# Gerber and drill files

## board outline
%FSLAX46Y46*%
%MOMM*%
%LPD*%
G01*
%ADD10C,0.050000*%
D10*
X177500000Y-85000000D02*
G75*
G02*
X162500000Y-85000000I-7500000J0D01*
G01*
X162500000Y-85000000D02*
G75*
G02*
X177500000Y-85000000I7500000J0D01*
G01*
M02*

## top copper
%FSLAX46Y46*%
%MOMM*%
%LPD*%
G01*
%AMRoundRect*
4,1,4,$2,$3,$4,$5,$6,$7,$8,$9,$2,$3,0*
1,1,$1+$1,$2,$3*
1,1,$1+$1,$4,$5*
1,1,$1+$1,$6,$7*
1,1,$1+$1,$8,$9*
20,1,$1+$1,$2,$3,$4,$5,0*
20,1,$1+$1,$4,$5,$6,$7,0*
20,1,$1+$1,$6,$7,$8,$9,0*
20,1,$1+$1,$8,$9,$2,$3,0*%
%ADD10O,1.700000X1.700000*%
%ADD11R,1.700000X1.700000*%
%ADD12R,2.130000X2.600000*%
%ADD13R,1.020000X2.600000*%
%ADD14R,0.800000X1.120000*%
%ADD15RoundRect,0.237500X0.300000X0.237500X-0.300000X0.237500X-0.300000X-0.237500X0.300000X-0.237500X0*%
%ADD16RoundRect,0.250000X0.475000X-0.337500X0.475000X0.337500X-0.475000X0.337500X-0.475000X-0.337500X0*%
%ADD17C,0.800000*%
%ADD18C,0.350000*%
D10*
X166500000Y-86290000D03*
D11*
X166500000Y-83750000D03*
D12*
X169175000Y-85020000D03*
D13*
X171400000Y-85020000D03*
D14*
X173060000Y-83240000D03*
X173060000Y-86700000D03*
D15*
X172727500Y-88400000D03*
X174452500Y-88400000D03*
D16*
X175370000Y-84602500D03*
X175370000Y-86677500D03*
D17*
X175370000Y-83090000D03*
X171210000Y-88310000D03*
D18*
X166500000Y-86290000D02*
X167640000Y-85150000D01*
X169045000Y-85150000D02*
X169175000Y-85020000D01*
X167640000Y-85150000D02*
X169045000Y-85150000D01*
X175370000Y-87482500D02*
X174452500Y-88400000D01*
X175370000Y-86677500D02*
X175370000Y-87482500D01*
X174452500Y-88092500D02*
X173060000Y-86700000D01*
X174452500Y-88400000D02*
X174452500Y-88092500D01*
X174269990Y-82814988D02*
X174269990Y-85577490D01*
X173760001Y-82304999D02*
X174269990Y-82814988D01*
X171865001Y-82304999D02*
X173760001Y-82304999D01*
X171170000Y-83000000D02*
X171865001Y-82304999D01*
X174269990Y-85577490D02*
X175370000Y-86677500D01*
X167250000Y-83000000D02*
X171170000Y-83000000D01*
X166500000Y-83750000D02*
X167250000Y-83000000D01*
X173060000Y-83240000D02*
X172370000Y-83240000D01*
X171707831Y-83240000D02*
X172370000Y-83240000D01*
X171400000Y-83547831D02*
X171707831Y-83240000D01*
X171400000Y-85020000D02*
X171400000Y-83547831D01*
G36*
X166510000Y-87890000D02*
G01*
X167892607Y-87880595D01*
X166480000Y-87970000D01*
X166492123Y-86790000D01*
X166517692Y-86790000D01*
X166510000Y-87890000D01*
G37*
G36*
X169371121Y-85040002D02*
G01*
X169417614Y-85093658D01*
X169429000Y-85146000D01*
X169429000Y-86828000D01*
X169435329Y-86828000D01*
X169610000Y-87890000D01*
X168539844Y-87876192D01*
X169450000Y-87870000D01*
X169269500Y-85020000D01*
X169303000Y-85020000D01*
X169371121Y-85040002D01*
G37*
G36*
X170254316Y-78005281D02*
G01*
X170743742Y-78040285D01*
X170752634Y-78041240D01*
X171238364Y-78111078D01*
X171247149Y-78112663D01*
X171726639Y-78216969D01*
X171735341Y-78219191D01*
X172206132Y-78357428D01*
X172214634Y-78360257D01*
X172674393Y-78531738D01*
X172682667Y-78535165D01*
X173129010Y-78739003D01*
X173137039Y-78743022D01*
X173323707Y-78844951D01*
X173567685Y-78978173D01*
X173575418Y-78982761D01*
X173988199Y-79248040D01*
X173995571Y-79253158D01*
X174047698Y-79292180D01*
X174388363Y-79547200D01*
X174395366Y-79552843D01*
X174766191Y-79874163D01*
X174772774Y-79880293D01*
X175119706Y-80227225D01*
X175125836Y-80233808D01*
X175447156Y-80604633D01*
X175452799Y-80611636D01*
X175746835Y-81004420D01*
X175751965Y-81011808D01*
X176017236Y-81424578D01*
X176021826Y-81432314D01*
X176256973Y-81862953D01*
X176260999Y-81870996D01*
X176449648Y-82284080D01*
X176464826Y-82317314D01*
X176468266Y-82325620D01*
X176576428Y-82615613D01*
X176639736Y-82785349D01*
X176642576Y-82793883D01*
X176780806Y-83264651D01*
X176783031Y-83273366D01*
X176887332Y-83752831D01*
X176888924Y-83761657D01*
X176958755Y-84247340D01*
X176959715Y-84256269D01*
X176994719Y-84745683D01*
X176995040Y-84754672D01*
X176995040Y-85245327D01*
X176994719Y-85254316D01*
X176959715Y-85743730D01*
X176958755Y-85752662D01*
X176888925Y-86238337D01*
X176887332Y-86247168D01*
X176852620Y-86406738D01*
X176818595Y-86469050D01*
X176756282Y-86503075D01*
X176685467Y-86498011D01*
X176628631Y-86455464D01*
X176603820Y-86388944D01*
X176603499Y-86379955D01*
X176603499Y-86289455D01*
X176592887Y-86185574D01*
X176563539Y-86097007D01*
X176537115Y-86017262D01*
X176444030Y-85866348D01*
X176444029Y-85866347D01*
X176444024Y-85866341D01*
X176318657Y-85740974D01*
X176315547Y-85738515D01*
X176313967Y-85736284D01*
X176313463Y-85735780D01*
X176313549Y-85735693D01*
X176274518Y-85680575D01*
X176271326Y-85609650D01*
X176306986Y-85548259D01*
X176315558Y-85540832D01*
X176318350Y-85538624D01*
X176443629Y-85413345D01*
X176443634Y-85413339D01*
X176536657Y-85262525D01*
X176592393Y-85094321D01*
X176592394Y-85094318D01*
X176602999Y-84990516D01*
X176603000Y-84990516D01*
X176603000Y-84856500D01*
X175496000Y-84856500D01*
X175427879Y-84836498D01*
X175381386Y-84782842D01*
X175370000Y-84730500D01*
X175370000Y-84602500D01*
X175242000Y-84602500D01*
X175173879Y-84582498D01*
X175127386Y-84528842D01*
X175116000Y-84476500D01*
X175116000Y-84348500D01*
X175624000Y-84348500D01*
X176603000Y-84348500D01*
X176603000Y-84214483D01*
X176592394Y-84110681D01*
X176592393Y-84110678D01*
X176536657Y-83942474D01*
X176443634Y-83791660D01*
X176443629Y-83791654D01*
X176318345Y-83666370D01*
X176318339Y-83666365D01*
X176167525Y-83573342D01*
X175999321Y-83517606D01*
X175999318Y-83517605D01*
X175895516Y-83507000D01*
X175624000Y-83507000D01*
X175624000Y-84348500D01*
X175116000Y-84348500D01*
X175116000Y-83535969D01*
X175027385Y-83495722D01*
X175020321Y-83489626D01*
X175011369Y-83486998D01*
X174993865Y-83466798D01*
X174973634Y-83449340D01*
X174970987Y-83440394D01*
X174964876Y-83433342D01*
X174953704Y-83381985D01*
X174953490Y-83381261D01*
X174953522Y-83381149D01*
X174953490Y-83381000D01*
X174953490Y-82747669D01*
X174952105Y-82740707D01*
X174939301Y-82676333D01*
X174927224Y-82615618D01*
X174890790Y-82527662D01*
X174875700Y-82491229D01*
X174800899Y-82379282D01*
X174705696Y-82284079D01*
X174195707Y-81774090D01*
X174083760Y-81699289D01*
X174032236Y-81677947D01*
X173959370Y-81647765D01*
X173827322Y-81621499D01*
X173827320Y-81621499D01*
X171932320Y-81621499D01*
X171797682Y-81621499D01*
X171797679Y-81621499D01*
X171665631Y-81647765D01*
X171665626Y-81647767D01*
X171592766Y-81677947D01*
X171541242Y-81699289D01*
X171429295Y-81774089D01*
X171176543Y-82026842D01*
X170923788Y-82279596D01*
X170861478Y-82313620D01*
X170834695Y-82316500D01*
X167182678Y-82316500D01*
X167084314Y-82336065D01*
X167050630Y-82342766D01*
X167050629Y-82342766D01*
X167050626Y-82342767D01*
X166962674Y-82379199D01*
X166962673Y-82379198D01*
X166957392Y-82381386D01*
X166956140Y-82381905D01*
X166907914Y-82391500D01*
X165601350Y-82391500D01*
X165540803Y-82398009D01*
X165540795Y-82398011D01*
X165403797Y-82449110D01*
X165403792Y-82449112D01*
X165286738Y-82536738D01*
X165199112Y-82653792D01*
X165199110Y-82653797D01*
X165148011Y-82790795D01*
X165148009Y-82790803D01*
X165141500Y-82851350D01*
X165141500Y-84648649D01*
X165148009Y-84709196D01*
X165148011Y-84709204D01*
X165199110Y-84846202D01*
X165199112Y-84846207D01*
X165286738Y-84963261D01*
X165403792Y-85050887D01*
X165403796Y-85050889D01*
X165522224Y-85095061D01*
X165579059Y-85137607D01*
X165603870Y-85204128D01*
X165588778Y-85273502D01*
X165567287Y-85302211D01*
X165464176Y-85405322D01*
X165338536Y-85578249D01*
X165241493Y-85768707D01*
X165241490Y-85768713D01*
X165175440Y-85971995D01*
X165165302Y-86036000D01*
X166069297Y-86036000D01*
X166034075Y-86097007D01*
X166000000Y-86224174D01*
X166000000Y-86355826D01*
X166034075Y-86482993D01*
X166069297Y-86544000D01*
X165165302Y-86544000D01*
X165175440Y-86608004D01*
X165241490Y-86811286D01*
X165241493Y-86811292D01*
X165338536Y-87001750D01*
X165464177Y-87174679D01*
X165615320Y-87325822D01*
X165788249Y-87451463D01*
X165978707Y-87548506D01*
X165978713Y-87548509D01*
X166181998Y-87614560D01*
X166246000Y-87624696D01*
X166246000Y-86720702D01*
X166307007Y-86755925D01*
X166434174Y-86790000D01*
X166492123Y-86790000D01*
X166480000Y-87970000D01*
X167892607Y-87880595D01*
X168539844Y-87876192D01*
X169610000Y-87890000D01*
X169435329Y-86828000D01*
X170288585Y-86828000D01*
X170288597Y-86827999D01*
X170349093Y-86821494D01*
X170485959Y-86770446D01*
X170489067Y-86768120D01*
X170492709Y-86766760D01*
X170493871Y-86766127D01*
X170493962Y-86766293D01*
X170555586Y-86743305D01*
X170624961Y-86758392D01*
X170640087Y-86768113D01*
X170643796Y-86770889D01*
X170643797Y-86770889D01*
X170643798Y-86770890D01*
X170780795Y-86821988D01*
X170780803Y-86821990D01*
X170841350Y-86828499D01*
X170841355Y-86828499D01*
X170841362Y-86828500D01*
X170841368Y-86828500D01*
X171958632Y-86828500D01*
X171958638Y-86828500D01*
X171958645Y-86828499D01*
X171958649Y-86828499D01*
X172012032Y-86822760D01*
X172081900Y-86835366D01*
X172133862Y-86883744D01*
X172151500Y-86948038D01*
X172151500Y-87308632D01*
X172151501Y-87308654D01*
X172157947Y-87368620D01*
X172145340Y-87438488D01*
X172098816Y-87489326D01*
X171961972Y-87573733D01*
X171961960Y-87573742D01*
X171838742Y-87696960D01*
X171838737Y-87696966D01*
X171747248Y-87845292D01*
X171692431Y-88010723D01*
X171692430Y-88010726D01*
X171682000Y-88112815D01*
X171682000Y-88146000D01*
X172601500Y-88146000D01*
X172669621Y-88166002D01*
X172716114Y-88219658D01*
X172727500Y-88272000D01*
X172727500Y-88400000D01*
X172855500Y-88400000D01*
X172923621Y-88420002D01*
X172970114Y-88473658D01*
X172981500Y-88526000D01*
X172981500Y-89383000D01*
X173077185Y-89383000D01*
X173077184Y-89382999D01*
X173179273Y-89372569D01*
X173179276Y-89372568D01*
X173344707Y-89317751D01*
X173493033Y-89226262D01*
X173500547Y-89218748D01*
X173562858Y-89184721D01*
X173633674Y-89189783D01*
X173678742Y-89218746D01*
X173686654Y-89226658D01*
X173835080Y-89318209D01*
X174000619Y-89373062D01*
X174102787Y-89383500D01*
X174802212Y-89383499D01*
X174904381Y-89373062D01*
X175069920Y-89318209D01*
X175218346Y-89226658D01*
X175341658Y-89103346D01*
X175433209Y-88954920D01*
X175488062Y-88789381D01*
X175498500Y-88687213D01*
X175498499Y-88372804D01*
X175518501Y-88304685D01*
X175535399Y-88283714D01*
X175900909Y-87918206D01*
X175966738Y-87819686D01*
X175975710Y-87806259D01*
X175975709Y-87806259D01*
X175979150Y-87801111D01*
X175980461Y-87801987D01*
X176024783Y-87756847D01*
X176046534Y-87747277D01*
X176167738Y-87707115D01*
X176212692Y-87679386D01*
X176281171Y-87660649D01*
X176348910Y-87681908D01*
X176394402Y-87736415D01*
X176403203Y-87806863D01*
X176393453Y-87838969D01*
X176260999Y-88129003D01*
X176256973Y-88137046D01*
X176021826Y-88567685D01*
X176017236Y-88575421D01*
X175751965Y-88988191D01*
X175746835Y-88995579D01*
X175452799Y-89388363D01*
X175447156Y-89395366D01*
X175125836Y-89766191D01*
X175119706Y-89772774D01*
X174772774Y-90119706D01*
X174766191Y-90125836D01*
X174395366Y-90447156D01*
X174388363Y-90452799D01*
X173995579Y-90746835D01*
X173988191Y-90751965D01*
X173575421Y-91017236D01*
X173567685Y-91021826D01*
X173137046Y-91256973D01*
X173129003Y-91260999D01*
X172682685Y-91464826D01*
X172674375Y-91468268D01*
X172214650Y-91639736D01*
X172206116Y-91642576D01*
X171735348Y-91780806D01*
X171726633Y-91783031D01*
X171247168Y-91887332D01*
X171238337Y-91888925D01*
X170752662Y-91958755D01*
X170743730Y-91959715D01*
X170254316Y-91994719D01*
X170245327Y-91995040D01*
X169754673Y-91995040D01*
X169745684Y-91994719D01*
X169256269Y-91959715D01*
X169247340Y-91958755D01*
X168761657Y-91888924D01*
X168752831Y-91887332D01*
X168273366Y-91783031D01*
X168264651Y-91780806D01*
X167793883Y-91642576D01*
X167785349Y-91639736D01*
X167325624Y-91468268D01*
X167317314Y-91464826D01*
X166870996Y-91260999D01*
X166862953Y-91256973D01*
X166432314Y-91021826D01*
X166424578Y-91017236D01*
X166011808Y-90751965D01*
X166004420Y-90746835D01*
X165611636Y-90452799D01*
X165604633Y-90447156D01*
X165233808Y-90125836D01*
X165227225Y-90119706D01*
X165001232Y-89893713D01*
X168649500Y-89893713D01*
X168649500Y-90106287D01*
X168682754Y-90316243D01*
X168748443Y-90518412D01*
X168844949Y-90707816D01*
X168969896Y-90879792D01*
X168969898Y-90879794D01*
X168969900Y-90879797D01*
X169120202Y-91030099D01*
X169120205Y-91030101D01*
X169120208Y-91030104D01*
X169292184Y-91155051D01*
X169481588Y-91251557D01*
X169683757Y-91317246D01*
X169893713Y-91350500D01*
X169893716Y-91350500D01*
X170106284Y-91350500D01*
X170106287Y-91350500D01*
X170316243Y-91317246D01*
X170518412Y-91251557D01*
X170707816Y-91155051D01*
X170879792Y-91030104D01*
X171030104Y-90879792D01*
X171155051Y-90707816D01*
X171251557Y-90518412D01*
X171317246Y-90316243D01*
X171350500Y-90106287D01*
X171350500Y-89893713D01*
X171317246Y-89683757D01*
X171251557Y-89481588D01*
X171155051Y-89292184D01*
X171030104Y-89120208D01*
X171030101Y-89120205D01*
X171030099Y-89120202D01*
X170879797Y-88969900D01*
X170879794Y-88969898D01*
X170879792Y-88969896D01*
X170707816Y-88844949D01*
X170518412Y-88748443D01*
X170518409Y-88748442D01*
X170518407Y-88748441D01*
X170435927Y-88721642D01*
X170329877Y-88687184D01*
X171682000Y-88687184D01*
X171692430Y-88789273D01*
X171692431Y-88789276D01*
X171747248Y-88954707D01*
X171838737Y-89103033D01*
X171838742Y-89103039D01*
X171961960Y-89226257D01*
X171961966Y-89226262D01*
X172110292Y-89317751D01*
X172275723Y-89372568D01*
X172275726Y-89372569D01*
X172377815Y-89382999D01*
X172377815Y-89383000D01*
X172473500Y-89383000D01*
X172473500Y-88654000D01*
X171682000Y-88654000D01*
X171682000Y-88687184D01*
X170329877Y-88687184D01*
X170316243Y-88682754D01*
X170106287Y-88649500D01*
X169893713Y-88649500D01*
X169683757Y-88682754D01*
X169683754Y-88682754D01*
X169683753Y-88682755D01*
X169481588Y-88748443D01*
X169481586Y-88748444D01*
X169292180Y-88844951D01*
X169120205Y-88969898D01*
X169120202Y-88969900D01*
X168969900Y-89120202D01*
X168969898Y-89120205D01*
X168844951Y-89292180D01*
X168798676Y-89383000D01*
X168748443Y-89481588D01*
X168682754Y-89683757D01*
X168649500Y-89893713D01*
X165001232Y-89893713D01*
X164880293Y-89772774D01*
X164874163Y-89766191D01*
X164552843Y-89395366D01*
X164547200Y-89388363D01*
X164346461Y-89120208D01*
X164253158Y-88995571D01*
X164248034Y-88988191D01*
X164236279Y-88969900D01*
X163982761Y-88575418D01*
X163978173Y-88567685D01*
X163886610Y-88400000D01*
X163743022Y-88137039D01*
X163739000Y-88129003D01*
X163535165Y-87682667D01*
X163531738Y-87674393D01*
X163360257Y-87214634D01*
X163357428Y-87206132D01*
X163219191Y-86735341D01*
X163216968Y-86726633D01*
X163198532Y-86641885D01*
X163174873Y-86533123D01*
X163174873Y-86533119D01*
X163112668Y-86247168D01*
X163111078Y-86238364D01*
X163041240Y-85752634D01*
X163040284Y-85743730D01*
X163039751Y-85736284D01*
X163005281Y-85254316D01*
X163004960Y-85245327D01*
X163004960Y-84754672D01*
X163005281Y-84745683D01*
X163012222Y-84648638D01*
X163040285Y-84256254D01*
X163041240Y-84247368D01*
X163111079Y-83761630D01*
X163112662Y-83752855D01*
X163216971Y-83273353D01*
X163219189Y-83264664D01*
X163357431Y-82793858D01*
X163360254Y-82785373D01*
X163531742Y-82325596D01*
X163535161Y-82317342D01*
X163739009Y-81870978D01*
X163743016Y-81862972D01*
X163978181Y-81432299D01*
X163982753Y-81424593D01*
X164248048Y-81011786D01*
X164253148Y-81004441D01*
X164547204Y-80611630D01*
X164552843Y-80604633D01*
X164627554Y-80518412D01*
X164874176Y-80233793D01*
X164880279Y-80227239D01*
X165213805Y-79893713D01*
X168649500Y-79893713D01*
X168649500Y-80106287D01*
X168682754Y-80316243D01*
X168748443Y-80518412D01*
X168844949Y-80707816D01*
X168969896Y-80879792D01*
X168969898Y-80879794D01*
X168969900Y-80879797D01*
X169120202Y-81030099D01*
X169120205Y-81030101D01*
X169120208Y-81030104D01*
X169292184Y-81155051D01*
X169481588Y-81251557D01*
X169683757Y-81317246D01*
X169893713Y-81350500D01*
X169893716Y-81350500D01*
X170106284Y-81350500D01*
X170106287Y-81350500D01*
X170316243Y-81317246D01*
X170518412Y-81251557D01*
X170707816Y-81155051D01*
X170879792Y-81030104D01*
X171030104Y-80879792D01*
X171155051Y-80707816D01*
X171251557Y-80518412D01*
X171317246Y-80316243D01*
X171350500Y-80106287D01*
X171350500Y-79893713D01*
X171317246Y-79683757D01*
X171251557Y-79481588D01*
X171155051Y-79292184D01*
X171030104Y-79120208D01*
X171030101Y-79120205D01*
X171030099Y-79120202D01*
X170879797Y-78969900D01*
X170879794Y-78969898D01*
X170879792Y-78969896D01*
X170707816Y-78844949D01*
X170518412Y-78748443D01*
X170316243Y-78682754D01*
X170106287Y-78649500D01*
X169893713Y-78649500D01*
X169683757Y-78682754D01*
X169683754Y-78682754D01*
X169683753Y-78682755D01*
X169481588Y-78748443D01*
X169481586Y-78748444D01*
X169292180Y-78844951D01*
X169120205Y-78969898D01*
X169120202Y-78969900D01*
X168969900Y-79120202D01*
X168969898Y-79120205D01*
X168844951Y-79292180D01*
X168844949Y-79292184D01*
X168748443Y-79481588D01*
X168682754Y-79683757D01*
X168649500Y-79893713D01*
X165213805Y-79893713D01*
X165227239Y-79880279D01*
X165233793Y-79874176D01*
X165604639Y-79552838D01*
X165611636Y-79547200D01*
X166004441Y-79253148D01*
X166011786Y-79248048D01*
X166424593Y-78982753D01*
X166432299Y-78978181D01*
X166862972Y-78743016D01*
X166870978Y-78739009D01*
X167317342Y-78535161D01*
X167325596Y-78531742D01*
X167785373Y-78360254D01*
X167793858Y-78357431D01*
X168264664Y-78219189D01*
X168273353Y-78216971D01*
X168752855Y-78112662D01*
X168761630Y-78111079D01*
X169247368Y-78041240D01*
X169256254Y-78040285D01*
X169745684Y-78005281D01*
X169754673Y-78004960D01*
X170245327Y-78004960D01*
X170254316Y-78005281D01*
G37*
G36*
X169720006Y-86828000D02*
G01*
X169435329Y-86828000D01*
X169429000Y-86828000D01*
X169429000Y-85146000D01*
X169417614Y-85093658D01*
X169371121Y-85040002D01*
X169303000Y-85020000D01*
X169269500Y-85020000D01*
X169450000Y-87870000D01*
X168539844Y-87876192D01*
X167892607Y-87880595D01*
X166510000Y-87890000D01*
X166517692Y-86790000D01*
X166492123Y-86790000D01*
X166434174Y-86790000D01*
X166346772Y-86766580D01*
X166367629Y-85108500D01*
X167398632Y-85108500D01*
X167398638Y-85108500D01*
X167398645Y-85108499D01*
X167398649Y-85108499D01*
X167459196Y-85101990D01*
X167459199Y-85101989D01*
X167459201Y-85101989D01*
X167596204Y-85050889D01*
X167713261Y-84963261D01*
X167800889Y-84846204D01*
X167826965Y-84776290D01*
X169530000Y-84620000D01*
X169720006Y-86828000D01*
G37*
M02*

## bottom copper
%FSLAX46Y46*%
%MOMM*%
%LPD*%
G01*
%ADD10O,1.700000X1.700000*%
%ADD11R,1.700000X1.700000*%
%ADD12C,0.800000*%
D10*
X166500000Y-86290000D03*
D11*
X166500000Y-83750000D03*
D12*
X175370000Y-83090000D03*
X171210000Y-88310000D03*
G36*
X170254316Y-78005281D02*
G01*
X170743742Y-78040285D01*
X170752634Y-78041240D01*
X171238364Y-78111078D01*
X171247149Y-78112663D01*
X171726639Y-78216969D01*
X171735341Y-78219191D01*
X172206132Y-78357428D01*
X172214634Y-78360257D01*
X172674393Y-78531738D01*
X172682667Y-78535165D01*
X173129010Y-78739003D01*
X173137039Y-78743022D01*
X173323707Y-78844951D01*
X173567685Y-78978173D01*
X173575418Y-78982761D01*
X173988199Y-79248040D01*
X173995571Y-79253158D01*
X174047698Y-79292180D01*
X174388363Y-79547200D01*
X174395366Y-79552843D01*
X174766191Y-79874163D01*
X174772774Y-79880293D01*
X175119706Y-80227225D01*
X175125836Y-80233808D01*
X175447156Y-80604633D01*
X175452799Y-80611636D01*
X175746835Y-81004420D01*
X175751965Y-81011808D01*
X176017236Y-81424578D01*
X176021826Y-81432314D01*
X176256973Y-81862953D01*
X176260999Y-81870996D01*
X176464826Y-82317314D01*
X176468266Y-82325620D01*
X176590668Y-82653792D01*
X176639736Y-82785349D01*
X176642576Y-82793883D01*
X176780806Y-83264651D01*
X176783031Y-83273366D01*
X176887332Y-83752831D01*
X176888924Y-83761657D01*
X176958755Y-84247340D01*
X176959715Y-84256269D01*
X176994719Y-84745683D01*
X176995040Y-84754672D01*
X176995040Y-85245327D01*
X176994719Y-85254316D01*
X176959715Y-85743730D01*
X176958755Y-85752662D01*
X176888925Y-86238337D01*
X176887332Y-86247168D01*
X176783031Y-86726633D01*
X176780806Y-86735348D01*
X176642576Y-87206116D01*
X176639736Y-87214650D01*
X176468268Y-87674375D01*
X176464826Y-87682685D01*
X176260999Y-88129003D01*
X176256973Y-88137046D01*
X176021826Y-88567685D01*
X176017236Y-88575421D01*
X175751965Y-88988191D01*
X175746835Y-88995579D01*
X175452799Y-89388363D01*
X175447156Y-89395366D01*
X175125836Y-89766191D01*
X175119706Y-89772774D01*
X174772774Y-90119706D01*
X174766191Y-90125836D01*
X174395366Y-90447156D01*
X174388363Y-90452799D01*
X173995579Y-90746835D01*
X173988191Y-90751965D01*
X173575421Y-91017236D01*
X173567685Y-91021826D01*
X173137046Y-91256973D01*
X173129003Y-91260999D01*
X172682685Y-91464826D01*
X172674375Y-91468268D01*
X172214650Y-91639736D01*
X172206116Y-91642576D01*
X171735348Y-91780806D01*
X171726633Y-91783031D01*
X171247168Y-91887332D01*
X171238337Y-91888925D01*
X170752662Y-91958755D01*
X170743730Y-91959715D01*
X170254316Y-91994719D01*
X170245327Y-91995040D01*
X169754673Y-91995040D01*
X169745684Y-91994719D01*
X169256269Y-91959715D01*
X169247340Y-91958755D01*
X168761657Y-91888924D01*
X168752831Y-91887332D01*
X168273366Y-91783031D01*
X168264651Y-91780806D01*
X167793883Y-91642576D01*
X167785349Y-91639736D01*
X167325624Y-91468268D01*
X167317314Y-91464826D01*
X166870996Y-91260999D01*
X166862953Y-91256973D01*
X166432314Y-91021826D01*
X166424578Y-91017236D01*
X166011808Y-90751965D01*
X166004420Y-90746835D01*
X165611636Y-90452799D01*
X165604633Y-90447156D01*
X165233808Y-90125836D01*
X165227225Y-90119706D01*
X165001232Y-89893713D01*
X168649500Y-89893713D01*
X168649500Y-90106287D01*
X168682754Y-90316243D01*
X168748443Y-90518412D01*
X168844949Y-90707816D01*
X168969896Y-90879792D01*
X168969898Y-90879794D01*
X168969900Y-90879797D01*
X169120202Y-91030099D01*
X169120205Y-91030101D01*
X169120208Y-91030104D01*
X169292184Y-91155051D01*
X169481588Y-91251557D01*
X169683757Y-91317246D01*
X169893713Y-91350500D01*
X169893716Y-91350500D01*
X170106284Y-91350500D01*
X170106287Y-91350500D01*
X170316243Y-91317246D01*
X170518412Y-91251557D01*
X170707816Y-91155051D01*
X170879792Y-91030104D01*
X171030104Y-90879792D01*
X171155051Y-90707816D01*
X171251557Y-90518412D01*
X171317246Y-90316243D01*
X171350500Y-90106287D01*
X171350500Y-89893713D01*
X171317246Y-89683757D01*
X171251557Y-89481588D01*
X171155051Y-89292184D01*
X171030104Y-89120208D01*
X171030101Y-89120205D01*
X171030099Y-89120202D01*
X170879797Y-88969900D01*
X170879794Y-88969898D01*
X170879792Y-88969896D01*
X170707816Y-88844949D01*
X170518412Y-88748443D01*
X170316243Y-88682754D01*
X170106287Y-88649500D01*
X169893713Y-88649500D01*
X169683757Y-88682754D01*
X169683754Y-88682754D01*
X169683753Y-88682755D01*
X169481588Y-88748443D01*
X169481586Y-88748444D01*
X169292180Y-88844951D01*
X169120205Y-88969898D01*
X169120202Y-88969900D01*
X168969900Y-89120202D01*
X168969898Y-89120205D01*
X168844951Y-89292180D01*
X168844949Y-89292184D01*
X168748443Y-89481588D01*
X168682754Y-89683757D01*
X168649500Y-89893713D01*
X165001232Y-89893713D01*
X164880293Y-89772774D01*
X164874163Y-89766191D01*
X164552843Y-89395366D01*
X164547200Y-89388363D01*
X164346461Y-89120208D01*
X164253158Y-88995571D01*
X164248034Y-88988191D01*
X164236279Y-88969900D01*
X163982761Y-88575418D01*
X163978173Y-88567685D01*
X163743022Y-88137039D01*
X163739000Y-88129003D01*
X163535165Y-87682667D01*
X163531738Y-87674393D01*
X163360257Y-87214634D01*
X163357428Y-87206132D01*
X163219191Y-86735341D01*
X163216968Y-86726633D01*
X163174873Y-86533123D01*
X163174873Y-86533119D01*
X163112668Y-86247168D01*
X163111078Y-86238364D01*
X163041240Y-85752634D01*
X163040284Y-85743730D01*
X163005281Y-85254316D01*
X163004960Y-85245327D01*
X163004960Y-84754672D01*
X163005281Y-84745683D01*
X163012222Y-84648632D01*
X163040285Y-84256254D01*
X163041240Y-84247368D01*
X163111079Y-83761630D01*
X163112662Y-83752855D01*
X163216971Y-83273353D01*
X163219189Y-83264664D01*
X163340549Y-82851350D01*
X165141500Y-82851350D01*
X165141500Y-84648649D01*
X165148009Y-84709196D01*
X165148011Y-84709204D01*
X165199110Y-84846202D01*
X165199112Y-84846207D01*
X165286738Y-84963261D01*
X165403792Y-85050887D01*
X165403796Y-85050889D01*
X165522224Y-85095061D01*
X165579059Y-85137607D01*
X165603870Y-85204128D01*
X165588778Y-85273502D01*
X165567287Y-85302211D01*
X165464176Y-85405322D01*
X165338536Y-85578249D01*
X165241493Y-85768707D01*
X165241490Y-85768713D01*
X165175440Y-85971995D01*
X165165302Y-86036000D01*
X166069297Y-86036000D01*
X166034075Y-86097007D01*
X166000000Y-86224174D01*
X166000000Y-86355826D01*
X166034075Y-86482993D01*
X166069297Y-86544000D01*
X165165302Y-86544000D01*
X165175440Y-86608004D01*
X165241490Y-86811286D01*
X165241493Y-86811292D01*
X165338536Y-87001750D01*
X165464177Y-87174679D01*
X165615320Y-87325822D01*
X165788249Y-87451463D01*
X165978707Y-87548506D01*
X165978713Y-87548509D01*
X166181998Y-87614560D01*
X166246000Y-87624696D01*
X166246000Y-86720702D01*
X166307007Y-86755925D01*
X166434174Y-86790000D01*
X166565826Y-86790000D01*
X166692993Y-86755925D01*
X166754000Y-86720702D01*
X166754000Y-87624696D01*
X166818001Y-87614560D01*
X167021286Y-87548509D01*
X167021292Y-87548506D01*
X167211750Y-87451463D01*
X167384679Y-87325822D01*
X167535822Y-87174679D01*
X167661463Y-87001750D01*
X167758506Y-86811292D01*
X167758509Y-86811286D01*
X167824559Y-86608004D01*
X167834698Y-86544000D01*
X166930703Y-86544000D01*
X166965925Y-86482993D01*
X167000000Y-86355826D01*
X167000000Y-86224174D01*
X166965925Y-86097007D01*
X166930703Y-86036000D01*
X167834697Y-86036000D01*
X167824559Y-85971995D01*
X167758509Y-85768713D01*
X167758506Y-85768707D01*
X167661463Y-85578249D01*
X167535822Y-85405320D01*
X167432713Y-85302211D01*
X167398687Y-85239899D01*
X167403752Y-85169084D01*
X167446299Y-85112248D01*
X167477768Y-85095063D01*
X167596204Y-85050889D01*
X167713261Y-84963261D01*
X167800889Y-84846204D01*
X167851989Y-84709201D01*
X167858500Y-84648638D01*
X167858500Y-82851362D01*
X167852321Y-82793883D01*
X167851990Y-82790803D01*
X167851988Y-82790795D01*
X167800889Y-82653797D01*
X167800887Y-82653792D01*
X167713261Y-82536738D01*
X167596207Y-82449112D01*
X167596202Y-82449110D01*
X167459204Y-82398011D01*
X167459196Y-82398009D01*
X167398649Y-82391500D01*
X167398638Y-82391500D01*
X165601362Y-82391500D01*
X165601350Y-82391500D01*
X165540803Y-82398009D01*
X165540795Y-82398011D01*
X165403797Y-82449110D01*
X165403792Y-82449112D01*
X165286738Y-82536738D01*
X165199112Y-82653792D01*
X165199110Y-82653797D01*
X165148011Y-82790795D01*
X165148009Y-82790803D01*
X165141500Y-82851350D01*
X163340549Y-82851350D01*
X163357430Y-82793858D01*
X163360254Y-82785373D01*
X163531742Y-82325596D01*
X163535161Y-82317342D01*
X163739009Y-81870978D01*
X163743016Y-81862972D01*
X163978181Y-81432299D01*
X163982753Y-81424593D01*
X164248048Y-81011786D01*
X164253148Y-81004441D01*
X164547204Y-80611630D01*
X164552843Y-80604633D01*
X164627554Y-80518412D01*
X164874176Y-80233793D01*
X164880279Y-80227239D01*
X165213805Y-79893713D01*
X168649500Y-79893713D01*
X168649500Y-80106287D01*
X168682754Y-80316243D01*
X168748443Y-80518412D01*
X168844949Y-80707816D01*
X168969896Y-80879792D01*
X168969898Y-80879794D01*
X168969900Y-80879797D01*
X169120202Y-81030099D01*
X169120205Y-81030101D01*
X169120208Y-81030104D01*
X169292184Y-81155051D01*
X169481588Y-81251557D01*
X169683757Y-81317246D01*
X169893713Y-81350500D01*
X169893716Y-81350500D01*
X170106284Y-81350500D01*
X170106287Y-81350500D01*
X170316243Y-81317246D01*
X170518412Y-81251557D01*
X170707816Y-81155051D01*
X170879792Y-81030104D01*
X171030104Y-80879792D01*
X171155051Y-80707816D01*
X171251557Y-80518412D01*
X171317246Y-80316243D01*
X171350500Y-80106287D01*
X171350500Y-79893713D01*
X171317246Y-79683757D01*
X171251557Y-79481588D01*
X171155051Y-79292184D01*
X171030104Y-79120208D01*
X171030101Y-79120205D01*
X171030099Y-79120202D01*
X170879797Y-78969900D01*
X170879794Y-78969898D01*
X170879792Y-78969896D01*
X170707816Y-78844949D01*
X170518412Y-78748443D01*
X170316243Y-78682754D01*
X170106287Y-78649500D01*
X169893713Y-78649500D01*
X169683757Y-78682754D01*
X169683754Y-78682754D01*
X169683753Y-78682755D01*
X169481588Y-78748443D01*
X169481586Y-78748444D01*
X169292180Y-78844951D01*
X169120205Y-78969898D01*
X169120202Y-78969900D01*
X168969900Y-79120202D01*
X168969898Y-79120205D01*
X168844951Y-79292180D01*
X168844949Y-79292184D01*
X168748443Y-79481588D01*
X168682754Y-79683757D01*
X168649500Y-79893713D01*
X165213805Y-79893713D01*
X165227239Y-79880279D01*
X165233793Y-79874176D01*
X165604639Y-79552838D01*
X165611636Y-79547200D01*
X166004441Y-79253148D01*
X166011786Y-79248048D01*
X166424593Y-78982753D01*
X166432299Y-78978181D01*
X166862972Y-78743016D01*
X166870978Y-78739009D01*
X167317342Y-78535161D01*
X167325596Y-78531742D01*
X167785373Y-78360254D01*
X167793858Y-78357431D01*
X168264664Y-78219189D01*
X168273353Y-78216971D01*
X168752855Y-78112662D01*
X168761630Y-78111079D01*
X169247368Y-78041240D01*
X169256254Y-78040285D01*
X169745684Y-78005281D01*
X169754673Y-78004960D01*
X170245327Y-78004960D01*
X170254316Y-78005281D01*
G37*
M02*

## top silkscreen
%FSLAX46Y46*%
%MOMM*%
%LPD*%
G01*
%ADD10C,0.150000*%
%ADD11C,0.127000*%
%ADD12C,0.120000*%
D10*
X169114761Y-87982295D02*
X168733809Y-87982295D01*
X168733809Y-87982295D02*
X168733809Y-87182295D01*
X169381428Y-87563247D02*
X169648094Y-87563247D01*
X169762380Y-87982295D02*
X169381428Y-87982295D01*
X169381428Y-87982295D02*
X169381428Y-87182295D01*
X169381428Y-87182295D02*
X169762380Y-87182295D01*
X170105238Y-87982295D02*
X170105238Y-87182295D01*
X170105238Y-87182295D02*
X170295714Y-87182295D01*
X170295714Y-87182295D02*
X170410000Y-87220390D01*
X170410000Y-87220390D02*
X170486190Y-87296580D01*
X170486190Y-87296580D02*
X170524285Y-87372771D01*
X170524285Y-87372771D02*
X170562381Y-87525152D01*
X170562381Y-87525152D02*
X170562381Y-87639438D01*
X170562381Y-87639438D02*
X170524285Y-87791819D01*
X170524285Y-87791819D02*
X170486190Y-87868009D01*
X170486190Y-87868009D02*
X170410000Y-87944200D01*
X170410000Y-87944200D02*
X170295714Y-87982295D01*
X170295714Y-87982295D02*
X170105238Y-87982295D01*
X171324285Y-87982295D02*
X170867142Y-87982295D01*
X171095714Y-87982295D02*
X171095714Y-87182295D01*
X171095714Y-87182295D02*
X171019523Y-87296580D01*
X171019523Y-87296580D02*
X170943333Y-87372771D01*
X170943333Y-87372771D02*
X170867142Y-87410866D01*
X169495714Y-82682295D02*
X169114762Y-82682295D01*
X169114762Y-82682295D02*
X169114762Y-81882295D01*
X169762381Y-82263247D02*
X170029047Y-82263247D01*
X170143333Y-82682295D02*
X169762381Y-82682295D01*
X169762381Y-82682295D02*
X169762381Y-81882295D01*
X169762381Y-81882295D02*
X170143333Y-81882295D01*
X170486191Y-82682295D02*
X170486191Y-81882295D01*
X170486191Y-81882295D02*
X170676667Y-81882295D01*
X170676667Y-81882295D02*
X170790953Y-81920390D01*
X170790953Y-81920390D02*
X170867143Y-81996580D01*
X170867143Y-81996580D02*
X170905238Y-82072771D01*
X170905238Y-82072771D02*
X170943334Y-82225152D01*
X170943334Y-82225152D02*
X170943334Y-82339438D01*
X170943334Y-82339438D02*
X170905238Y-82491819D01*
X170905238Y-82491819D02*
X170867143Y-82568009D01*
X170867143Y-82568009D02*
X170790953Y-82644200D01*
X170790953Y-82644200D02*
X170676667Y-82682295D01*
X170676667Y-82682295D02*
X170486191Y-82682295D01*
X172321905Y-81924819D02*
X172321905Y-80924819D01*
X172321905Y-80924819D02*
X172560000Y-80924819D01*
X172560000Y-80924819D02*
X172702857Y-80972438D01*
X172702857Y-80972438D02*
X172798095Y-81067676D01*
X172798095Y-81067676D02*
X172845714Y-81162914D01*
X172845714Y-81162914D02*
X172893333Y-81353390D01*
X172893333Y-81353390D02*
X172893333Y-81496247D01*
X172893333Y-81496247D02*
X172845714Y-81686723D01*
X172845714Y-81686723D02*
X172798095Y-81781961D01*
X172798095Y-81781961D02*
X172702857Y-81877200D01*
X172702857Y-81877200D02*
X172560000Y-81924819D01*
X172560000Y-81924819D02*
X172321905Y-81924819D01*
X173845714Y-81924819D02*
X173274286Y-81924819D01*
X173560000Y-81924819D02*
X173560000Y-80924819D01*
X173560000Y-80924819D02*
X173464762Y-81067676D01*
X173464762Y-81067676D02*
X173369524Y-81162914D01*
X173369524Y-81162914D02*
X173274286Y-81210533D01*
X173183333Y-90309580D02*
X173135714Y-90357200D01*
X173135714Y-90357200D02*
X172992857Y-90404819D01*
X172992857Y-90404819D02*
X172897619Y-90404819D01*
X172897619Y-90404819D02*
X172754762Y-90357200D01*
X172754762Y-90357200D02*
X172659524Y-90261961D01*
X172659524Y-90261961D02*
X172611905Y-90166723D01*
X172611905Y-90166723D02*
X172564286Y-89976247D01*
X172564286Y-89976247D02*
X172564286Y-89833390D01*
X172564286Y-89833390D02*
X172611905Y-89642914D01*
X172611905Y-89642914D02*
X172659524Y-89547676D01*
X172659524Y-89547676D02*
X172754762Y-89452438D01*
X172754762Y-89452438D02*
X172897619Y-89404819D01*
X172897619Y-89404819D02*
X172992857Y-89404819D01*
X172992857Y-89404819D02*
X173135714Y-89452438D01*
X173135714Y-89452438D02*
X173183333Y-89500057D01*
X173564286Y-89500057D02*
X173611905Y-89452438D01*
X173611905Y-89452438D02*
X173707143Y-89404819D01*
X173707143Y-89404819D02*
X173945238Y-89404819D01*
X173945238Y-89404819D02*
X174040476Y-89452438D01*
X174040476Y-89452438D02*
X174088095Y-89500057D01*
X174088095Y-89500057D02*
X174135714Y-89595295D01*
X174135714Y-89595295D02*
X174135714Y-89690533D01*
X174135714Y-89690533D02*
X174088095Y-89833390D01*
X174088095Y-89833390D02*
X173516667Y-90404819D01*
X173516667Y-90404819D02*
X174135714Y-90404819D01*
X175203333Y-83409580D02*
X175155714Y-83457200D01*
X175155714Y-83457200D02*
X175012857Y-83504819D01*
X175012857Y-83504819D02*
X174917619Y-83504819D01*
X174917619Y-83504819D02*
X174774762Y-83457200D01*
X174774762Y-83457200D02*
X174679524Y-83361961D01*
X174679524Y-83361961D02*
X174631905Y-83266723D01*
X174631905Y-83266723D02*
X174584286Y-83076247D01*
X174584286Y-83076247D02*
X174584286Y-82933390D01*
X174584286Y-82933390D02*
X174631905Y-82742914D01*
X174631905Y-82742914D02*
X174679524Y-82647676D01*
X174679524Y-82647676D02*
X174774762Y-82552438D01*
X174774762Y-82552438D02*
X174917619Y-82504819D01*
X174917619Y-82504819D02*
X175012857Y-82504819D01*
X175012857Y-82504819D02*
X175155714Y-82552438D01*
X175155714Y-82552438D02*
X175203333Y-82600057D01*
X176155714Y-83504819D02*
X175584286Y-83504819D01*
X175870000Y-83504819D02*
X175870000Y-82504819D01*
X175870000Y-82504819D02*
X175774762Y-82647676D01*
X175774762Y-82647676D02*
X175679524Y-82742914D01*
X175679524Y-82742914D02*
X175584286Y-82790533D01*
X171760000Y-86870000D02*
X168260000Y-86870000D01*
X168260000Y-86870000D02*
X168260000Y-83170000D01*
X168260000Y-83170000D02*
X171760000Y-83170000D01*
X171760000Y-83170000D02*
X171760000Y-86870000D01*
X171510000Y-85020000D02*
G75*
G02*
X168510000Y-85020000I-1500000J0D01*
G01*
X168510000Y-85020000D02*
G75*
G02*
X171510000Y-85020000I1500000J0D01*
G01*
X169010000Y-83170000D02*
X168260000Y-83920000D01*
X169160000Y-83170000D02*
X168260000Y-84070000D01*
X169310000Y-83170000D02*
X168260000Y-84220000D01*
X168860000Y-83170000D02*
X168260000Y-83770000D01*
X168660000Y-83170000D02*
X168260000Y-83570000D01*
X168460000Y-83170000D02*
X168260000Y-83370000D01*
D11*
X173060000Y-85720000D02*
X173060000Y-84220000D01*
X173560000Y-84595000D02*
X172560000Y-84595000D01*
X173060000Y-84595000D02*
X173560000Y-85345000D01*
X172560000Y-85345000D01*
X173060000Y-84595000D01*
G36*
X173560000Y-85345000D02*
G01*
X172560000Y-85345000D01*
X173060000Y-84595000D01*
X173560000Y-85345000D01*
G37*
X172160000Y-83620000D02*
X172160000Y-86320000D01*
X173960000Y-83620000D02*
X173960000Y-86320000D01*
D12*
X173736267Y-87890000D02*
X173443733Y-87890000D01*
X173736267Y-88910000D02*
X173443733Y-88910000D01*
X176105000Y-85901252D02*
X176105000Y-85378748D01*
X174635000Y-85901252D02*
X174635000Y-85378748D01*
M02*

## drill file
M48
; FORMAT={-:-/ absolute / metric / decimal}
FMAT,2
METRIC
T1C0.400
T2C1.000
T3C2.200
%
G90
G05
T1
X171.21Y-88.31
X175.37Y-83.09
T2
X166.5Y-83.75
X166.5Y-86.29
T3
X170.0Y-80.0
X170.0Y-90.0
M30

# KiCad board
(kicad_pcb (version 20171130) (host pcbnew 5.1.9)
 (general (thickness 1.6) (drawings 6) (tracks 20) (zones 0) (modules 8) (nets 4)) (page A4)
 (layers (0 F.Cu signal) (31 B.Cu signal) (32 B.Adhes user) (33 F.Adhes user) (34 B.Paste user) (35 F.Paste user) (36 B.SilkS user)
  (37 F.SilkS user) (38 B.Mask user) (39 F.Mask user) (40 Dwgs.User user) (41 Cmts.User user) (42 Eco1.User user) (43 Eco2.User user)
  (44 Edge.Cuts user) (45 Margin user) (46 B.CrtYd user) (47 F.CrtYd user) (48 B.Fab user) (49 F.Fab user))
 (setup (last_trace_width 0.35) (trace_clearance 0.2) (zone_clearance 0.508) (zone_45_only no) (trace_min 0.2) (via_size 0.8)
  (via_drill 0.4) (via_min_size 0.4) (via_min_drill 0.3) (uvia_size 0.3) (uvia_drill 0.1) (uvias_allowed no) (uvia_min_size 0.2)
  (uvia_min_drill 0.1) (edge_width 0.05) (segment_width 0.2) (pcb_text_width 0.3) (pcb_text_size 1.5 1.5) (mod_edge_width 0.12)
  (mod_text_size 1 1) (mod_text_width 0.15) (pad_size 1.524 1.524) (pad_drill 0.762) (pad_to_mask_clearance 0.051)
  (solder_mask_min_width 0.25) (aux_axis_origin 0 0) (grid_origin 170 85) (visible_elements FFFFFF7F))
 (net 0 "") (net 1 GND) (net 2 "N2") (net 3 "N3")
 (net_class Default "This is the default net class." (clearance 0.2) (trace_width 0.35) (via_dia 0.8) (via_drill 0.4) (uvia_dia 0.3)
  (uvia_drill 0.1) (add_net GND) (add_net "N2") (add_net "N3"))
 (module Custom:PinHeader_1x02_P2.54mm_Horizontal (layer B.Cu) (at 166.5 83.75 180)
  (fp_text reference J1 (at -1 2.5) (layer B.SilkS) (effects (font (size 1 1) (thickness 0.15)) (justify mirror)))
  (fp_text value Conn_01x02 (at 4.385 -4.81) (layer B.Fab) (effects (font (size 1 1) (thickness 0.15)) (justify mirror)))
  (pad 2 thru_hole oval (at 0 -2.54 180) (size 1.7 1.7) (drill 1) (layers *.Cu *.Mask) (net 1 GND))
  (pad 1 thru_hole rect (at 0 0 180) (size 1.7 1.7) (drill 1) (layers *.Cu *.Mask) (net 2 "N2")))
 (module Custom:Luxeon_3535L (layer F.Cu) (at 170.01 85.02 180)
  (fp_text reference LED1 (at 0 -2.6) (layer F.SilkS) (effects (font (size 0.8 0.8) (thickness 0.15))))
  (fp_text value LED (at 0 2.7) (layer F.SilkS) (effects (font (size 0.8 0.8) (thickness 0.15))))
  (fp_line (start -1.75 -1.85) (end 1.75 -1.85) (layer F.SilkS) (width 0.15))
  (fp_line (start 1.75 -1.85) (end 1.75 1.85) (layer F.SilkS) (width 0.15))
  (fp_line (start 1.75 1.85) (end -1.75 1.85) (layer F.SilkS) (width 0.15))
  (fp_line (start -1.75 1.85) (end -1.75 -1.85) (layer F.SilkS) (width 0.15))
  (fp_circle (center 0 0) (end 1.5 0) (layer F.SilkS) (width 0.15))
  (fp_line (start 1 1.85) (end 1.75 1.1) (layer F.SilkS) (width 0.15))
  (fp_line (start 0.85 1.85) (end 1.75 0.95) (layer F.SilkS) (width 0.15))
  (fp_line (start 0.7 1.85) (end 1.75 0.8) (layer F.SilkS) (width 0.15))
  (fp_line (start 1.15 1.85) (end 1.75 1.25) (layer F.SilkS) (width 0.15))
  (fp_line (start 1.35 1.85) (end 1.75 1.45) (layer F.SilkS) (width 0.15))
  (fp_line (start 1.55 1.85) (end 1.75 1.65) (layer F.SilkS) (width 0.15))
  (pad 1 smd rect (at 0.835 0 180) (size 2.13 2.6) (layers F.Cu F.Paste F.Mask) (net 1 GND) (solder_paste_margin -0.05))
  (pad 2 smd rect (at -1.39 0 180) (size 1.02 2.6) (layers F.Cu F.Paste F.Mask) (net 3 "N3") (solder_paste_margin -0.05)))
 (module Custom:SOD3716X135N (layer F.Cu) (at 173.06 84.97 270)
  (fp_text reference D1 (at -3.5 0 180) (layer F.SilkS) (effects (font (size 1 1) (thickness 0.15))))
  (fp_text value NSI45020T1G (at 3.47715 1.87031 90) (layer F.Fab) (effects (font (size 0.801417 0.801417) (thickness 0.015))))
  (fp_line (start 0.75 0) (end -0.75 0) (layer F.SilkS) (width 0.127))
  (fp_line (start -0.375 -0.5) (end -0.375 0.5) (layer F.SilkS) (width 0.127))
  (fp_poly (pts (xy -0.375 0) (xy 0.375 -0.5) (xy 0.375 0.5)) (layer F.SilkS) (width 0.127))
  (fp_line (start -1.35 0.9) (end 1.35 0.9) (layer F.SilkS) (width 0.127))
  (fp_line (start -1.35 -0.9) (end 1.35 -0.9) (layer F.SilkS) (width 0.127))
  (pad 1 smd rect (at -1.73 0 270) (size 1.12 0.8) (layers F.Cu F.Paste F.Mask) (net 3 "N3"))
  (pad 2 smd rect (at 1.73 0 270) (size 1.12 0.8) (layers F.Cu F.Paste F.Mask) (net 2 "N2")))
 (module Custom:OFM (layer B.Cu) (at 170 85 270)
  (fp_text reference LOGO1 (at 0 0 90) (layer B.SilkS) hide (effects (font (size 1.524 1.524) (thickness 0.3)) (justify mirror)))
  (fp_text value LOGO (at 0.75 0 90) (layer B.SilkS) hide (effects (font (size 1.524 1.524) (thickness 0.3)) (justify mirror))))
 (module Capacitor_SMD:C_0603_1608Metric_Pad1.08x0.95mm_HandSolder (layer F.Cu) (at 173.59 88.4 180)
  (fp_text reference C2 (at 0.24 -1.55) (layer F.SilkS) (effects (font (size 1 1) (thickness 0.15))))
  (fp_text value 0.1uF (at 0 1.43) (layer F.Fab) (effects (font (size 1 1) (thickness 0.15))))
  (fp_line (start -0.146267 0.51) (end 0.146267 0.51) (layer F.SilkS) (width 0.12))
  (fp_line (start -0.146267 -0.51) (end 0.146267 -0.51) (layer F.SilkS) (width 0.12))
  (pad 2 smd roundrect (at 0.8625 0 180) (size 1.075 0.95) (layers F.Cu F.Paste F.Mask) (roundrect_rratio 0.25) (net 1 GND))
  (pad 1 smd roundrect (at -0.8625 0 180) (size 1.075 0.95) (layers F.Cu F.Paste F.Mask) (roundrect_rratio 0.25) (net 2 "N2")))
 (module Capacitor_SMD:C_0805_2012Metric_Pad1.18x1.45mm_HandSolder (layer F.Cu) (at 175.37 85.64 90)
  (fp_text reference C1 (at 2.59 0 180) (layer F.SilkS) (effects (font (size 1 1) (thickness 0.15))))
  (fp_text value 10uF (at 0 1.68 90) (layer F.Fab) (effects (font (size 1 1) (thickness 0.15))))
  (fp_line (start -0.261252 0.735) (end 0.261252 0.735) (layer F.SilkS) (width 0.12))
  (fp_line (start -0.261252 -0.735) (end 0.261252 -0.735) (layer F.SilkS) (width 0.12))
  (pad 2 smd roundrect (at 1.0375 0 90) (size 1.175 1.45) (layers F.Cu F.Paste F.Mask) (roundrect_rratio 0.2127659574468085) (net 1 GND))
  (pad 1 smd roundrect (at -1.0375 0 90) (size 1.175 1.45) (layers F.Cu F.Paste F.Mask) (roundrect_rratio 0.2127659574468085) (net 2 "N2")))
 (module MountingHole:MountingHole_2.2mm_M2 (layer B.Cu) (at 170 90)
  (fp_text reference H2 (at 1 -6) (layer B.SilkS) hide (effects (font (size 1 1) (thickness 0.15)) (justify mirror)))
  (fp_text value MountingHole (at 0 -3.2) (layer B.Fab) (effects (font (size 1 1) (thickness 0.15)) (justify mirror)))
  (pad 1 np_thru_hole circle (at 0 0) (size 2.2 2.2) (drill 2.2) (layers *.Cu *.Mask)))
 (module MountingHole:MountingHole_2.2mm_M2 (layer B.Cu) (at 170 80)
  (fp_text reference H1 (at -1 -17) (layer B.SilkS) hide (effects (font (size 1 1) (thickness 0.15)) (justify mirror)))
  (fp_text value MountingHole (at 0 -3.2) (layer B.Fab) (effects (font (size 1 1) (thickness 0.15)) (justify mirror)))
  (pad 1 np_thru_hole circle (at 0 0) (size 2.2 2.2) (drill 2.2) (layers *.Cu *.Mask)))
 (gr_circle (center 170 85) (end 177.5 85) (layer Edge.Cuts) (width 0.05))
 (via (at 175.37 83.09) (size 0.8) (drill 0.4) (layers F.Cu B.Cu) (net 1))
 (via (at 171.21 88.31) (size 0.8) (drill 0.4) (layers F.Cu B.Cu) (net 1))
 (segment (start 166.5 86.29) (end 167.64 85.15) (width 0.35) (layer F.Cu) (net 1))
 (segment (start 169.045 85.15) (end 169.175 85.02) (width 0.35) (layer F.Cu) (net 1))
 (segment (start 167.64 85.15) (end 169.045 85.15) (width 0.35) (layer F.Cu) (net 1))
 (segment (start 175.37 87.4825) (end 174.4525 88.4) (width 0.35) (layer F.Cu) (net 2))
 (segment (start 175.37 86.6775) (end 175.37 87.4825) (width 0.35) (layer F.Cu) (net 2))
 (segment (start 174.4525 88.0925) (end 173.06 86.7) (width 0.35) (layer F.Cu) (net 2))
 (segment (start 174.4525 88.4) (end 174.4525 88.0925) (width 0.35) (layer F.Cu) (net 2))
 (segment (start 174.26999 82.814988) (end 174.26999 85.57749) (width 0.35) (layer F.Cu) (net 2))
 (segment (start 173.760001 82.304999) (end 174.26999 82.814988) (width 0.35) (layer F.Cu) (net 2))
 (segment (start 171.865001 82.304999) (end 173.760001 82.304999) (width 0.35) (layer F.Cu) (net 2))
 (segment (start 171.17 83) (end 171.865001 82.304999) (width 0.35) (layer F.Cu) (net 2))
 (segment (start 174.26999 85.57749) (end 175.37 86.6775) (width 0.35) (layer F.Cu) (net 2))
 (segment (start 167.25 83) (end 171.17 83) (width 0.35) (layer F.Cu) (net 2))
 (segment (start 166.5 83.75) (end 167.25 83) (width 0.35) (layer F.Cu) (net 2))
 (segment (start 173.06 83.24) (end 172.37 83.24) (width 0.35) (layer F.Cu) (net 3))
 (segment (start 171.707831 83.24) (end 172.37 83.24) (width 0.35) (layer F.Cu) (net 3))
 (segment (start 171.4 83.547831) (end 171.707831 83.24) (width 0.35) (layer F.Cu) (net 3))
 (segment (start 171.4 85.02) (end 171.4 83.547831) (width 0.35) (layer F.Cu) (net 3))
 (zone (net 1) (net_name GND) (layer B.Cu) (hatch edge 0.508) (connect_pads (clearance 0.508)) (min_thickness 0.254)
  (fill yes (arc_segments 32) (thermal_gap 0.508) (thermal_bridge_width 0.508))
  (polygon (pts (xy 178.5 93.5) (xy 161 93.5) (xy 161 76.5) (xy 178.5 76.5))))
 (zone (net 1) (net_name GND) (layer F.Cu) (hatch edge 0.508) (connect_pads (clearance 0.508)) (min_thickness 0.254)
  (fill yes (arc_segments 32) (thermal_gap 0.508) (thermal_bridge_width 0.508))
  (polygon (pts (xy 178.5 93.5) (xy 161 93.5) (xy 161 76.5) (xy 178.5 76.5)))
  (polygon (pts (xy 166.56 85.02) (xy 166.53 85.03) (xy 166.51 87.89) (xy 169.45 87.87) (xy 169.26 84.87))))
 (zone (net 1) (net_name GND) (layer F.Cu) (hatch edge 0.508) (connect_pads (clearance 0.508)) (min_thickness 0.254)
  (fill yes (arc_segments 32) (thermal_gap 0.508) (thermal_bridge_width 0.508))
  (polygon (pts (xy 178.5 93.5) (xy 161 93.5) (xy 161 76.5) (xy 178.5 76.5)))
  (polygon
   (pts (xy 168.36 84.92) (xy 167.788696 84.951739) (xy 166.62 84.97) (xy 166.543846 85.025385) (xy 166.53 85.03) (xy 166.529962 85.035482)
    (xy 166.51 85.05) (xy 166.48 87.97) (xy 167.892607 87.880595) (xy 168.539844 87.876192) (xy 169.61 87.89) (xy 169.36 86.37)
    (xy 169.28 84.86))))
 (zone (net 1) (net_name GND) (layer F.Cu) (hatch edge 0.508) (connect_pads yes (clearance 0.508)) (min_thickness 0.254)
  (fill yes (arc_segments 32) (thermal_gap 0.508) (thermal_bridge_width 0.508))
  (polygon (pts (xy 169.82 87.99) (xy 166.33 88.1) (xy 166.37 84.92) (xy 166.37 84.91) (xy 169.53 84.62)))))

